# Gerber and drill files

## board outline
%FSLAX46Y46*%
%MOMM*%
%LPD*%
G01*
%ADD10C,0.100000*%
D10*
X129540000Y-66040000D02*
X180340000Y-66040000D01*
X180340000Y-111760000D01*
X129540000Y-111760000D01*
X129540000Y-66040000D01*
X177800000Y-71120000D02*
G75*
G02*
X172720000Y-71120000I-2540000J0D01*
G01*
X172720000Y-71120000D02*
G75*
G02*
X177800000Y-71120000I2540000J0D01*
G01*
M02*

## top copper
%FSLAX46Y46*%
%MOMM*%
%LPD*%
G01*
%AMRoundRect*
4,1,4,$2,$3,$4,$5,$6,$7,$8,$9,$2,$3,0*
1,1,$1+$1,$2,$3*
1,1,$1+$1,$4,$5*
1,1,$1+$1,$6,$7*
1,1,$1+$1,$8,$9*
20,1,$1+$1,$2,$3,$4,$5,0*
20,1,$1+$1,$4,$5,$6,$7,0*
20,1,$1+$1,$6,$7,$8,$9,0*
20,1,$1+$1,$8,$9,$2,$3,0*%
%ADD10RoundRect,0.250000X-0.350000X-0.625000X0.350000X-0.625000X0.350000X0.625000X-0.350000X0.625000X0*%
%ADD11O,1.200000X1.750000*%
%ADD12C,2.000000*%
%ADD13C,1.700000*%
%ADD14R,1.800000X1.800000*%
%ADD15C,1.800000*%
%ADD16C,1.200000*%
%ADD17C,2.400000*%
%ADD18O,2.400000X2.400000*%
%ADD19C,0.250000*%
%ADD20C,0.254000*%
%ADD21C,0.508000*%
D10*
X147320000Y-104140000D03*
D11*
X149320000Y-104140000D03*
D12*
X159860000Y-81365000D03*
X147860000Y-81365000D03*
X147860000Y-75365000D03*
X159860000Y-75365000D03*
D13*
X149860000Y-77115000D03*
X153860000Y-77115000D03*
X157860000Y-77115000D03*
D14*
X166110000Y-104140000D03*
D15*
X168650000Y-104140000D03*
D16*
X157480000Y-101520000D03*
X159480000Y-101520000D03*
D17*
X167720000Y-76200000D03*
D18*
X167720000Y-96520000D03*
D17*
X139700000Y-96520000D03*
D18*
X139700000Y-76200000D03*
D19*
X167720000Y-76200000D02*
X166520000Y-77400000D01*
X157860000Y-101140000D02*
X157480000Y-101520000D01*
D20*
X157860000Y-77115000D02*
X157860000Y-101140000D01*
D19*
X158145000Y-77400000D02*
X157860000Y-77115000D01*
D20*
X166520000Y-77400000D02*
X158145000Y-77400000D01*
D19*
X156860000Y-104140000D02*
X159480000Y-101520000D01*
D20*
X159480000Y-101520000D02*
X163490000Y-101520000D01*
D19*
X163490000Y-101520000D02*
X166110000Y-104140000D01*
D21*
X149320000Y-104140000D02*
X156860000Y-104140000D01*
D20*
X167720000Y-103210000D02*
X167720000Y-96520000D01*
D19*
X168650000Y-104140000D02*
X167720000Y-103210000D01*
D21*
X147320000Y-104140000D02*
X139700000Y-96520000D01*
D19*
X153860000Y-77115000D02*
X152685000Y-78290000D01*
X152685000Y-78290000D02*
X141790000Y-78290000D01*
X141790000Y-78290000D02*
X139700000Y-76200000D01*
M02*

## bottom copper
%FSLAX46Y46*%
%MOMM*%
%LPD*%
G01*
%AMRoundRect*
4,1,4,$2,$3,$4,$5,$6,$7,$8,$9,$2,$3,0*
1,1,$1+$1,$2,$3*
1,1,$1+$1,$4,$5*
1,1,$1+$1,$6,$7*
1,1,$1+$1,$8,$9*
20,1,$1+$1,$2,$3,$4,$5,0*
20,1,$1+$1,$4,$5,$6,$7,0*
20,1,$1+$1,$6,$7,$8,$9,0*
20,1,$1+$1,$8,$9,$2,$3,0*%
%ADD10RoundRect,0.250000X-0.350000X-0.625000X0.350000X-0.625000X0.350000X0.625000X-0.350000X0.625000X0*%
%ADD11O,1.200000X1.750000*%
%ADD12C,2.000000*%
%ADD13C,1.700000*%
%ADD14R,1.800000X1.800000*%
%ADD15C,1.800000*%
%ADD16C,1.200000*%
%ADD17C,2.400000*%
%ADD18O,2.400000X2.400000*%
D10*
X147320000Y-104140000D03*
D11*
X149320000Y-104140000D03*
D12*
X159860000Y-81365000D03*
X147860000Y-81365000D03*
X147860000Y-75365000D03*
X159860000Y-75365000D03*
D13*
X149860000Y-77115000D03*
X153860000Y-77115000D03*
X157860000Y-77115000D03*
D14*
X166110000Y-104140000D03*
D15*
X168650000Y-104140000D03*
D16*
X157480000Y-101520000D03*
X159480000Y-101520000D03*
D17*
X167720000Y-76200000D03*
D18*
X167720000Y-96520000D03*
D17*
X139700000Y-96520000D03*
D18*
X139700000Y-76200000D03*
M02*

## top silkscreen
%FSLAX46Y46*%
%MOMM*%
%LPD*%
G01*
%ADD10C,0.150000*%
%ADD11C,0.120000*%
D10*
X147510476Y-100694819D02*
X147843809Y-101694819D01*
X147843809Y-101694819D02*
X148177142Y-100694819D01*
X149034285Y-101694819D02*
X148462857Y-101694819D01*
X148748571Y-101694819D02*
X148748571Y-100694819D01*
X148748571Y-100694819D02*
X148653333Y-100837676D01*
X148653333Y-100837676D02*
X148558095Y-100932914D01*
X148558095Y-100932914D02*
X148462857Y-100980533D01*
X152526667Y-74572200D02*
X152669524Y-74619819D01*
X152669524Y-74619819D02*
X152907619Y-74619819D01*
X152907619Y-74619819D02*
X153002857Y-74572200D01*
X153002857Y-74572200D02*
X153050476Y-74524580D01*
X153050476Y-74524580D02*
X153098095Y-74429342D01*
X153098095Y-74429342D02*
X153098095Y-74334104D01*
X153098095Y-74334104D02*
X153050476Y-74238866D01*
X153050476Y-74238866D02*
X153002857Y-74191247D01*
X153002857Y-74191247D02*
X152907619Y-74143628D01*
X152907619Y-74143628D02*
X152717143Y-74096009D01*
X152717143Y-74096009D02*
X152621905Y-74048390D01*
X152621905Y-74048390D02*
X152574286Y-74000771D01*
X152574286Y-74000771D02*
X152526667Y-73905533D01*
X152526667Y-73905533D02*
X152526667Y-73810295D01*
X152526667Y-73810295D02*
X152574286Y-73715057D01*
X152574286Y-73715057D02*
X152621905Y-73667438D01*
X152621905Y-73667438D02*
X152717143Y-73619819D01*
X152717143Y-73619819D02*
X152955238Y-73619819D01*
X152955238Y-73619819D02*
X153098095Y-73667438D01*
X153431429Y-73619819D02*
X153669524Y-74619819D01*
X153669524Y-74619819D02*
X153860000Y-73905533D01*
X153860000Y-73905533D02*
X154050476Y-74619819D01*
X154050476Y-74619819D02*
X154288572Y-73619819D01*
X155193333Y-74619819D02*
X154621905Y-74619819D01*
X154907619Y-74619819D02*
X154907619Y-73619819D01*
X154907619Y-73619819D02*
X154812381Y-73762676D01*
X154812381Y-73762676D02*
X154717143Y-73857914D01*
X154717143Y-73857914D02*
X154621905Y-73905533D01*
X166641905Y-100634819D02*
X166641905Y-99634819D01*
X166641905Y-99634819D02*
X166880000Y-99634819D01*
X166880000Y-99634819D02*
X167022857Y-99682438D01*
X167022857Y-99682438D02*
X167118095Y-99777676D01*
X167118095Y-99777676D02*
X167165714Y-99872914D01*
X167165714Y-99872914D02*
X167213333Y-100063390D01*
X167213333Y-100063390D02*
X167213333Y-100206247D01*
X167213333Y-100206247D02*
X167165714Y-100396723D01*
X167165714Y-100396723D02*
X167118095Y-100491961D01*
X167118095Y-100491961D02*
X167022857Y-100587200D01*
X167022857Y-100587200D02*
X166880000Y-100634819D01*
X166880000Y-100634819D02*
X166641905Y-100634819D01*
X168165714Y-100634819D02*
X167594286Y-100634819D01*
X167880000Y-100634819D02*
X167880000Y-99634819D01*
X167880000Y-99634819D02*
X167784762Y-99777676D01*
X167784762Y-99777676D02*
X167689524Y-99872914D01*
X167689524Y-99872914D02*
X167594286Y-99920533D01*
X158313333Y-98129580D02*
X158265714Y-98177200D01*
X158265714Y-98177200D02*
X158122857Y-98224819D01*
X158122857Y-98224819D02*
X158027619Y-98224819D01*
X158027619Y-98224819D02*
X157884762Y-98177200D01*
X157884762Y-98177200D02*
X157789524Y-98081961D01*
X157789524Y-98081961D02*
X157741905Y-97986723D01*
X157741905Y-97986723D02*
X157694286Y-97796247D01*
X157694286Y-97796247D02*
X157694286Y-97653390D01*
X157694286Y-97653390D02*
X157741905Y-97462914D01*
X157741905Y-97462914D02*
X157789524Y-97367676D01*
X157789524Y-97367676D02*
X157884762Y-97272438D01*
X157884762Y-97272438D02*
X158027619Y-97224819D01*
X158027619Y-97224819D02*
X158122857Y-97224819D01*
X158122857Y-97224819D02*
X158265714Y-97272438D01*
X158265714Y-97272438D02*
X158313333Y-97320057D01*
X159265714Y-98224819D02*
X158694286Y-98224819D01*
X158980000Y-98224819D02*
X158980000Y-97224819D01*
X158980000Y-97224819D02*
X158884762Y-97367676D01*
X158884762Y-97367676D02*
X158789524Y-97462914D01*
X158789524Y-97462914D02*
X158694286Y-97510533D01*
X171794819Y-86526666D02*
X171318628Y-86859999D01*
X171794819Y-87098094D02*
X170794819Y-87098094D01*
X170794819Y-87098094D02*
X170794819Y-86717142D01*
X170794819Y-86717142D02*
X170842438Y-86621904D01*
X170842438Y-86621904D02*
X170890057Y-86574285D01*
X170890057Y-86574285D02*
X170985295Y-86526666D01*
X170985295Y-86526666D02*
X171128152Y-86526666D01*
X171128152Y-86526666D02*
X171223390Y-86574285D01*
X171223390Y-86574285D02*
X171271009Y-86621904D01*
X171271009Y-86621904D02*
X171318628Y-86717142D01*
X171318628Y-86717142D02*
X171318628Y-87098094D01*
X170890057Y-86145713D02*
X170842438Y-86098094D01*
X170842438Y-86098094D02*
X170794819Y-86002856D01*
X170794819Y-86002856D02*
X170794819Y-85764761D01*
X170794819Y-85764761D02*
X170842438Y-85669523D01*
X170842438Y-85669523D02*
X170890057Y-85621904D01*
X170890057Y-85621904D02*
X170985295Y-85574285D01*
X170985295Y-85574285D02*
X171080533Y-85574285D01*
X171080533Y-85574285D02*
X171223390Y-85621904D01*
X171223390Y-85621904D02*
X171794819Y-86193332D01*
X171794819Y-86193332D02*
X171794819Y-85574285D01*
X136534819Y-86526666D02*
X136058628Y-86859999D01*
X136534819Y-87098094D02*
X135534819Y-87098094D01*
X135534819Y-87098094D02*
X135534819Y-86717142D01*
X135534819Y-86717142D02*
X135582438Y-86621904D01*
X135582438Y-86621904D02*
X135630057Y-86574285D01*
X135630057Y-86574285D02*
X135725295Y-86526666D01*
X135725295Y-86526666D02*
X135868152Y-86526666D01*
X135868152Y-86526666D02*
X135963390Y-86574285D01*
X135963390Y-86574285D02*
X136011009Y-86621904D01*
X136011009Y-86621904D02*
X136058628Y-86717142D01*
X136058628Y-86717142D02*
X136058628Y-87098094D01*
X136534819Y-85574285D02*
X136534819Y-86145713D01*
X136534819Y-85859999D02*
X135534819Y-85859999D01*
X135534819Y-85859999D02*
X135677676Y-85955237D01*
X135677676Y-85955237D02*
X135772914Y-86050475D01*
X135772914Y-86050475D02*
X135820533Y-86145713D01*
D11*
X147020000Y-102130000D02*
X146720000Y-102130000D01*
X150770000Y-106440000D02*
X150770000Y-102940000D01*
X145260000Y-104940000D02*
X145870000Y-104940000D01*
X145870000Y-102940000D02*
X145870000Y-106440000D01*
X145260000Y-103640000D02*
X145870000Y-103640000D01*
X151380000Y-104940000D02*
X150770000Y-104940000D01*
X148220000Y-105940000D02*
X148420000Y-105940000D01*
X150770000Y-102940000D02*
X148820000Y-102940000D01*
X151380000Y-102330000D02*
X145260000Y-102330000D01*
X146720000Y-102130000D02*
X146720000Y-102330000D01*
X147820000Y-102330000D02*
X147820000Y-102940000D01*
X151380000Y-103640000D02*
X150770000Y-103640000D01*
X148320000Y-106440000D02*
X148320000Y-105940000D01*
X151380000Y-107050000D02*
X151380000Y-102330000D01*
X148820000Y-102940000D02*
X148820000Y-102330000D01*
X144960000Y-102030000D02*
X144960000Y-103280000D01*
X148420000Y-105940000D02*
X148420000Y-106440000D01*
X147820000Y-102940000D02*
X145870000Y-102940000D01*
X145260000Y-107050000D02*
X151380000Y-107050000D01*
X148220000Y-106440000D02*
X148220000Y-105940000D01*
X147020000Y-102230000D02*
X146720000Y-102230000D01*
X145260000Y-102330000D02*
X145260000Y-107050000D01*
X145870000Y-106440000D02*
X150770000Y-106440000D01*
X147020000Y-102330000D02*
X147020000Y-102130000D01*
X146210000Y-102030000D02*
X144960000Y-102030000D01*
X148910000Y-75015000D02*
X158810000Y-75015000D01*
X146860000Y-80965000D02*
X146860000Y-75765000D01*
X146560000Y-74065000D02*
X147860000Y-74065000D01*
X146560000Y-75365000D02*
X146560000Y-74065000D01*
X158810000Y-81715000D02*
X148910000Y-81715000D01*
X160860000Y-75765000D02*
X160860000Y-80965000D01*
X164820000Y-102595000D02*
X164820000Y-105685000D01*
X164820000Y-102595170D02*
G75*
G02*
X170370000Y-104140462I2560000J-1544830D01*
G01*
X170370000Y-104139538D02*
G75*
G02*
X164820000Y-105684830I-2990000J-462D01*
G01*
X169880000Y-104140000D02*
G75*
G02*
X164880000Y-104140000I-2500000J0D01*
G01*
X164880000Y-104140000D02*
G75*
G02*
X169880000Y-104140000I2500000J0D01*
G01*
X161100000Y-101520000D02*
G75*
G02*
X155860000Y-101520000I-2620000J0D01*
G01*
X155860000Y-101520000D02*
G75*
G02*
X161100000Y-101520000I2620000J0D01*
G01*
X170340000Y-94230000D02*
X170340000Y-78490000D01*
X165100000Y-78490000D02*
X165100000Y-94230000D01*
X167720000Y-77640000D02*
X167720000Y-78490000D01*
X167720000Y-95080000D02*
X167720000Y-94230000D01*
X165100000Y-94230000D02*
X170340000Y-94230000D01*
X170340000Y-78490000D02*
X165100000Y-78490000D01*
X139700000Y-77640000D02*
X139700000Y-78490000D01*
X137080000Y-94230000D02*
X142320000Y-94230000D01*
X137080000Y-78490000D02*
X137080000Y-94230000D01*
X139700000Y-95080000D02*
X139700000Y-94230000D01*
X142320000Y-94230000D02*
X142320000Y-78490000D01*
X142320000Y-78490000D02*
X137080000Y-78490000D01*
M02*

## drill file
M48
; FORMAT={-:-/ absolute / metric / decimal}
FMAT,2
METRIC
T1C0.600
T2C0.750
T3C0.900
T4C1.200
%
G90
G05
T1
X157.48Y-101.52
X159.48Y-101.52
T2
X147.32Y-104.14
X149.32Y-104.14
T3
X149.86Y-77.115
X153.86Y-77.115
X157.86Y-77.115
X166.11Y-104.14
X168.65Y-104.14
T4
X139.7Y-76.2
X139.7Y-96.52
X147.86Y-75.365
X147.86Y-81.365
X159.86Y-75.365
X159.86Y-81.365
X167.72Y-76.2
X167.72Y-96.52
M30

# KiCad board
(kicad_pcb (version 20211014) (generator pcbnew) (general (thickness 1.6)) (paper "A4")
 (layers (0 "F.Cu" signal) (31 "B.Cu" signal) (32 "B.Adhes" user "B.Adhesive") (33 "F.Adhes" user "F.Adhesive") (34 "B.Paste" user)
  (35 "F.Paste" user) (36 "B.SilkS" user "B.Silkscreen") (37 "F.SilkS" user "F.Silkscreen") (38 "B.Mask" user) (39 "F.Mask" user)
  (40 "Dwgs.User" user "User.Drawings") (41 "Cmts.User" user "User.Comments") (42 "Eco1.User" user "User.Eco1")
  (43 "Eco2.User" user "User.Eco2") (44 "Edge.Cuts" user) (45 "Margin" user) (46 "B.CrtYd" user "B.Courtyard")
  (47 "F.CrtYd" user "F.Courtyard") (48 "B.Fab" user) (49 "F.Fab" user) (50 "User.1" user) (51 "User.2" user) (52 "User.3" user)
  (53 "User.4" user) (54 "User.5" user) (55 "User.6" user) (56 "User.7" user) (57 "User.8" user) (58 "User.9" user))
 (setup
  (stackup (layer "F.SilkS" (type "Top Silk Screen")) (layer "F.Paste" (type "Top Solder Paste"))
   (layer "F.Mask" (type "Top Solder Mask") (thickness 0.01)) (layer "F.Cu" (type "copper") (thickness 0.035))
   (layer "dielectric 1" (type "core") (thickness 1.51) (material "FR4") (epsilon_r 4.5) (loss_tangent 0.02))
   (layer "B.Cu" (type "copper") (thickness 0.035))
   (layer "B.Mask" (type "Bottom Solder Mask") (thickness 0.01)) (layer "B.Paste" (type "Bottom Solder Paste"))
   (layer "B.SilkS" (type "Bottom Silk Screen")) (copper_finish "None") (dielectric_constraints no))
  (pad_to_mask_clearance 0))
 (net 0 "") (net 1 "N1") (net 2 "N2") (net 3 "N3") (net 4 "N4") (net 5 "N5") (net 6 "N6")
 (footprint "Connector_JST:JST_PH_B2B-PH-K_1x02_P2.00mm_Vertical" (layer "F.Cu") (at 147.32 104.14)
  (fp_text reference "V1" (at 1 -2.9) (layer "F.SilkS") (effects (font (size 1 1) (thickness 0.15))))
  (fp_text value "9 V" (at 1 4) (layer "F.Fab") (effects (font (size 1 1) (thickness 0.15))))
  (fp_line (start -0.3 -2.01) (end -0.6 -2.01) (layer "F.SilkS") (width 0.12))
  (fp_line (start 3.45 2.3) (end 3.45 -1.2) (layer "F.SilkS") (width 0.12))
  (fp_line (start -2.06 0.8) (end -1.45 0.8) (layer "F.SilkS") (width 0.12))
  (fp_line (start -1.45 -1.2) (end -1.45 2.3) (layer "F.SilkS") (width 0.12))
  (fp_line (start -2.06 -0.5) (end -1.45 -0.5) (layer "F.SilkS") (width 0.12))
  (fp_line (start 4.06 0.8) (end 3.45 0.8) (layer "F.SilkS") (width 0.12))
  (fp_line (start 0.9 1.8) (end 1.1 1.8) (layer "F.SilkS") (width 0.12))
  (fp_line (start 3.45 -1.2) (end 1.5 -1.2) (layer "F.SilkS") (width 0.12))
  (fp_line (start 4.06 -1.81) (end -2.06 -1.81) (layer "F.SilkS") (width 0.12))
  (fp_line (start -0.6 -2.01) (end -0.6 -1.81) (layer "F.SilkS") (width 0.12))
  (fp_line (start 0.5 -1.81) (end 0.5 -1.2) (layer "F.SilkS") (width 0.12))
  (fp_line (start 4.06 -0.5) (end 3.45 -0.5) (layer "F.SilkS") (width 0.12))
  (fp_line (start 1 2.3) (end 1 1.8) (layer "F.SilkS") (width 0.12))
  (fp_line (start 4.06 2.91) (end 4.06 -1.81) (layer "F.SilkS") (width 0.12))
  (fp_line (start 1.5 -1.2) (end 1.5 -1.81) (layer "F.SilkS") (width 0.12))
  (fp_line (start -2.36 -2.11) (end -2.36 -0.86) (layer "F.SilkS") (width 0.12))
  (fp_line (start 1.1 1.8) (end 1.1 2.3) (layer "F.SilkS") (width 0.12))
  (fp_line (start 0.5 -1.2) (end -1.45 -1.2) (layer "F.SilkS") (width 0.12))
  (fp_line (start -2.06 2.91) (end 4.06 2.91) (layer "F.SilkS") (width 0.12))
  (fp_line (start 0.9 2.3) (end 0.9 1.8) (layer "F.SilkS") (width 0.12))
  (fp_line (start -0.3 -1.91) (end -0.6 -1.91) (layer "F.SilkS") (width 0.12))
  (fp_line (start -2.06 -1.81) (end -2.06 2.91) (layer "F.SilkS") (width 0.12))
  (fp_line (start -1.45 2.3) (end 3.45 2.3) (layer "F.SilkS") (width 0.12))
  (fp_line (start -0.3 -1.81) (end -0.3 -2.01) (layer "F.SilkS") (width 0.12))
  (fp_line (start -1.11 -2.11) (end -2.36 -2.11) (layer "F.SilkS") (width 0.12))
  (pad "1" thru_hole roundrect (at 0 0) (size 1.2 1.75) (drill 0.75) (layers *.Cu *.Mask) (roundrect_rratio 0.208333) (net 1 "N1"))
  (pad "2" thru_hole oval (at 2 0) (size 1.2 1.75) (drill 0.75) (layers *.Cu *.Mask) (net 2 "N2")))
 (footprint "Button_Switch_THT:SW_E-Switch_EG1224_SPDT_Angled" (layer "F.Cu") (at 149.86 77.115)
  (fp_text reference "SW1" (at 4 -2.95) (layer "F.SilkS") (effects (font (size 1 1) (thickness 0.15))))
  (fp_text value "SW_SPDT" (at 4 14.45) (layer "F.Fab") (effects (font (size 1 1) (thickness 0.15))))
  (fp_line (start -0.95 -2.1) (end 8.95 -2.1) (layer "F.SilkS") (width 0.12))
  (fp_line (start -3 3.85) (end -3 -1.35) (layer "F.SilkS") (width 0.12))
  (fp_line (start -3.3 -3.05) (end -2 -3.05) (layer "F.SilkS") (width 0.12))
  (fp_line (start -3.3 -1.75) (end -3.3 -3.05) (layer "F.SilkS") (width 0.12))
  (fp_line (start 8.95 4.6) (end -0.95 4.6) (layer "F.SilkS") (width 0.12))
  (fp_line (start 11 -1.35) (end 11 3.85) (layer "F.SilkS") (width 0.12))
  (pad "" thru_hole circle (at 10 4.25) (size 2 2) (drill 1.2) (layers *.Cu *.Mask))
  (pad "" thru_hole circle (at -2 4.25) (size 2 2) (drill 1.2) (layers *.Cu *.Mask))
  (pad "" thru_hole circle (at -2 -1.75) (size 2 2) (drill 1.2) (layers *.Cu *.Mask))
  (pad "" thru_hole circle (at 10 -1.75) (size 2 2) (drill 1.2) (layers *.Cu *.Mask))
  (pad "1" thru_hole circle (at 0 0) (size 1.7 1.7) (drill 0.9) (layers *.Cu *.Mask) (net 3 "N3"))
  (pad "2" thru_hole circle (at 4 0) (size 1.7 1.7) (drill 0.9) (layers *.Cu *.Mask) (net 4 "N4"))
  (pad "3" thru_hole circle (at 8 0) (size 1.7 1.7) (drill 0.9) (layers *.Cu *.Mask) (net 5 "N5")))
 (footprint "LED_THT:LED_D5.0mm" (layer "F.Cu") (at 166.11 104.14)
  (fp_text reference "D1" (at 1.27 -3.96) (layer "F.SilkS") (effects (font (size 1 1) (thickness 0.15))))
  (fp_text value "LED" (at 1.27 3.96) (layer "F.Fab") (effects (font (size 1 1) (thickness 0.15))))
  (fp_line (start -1.29 -1.545) (end -1.29 1.545) (layer "F.SilkS") (width 0.12))
  (fp_arc (start -1.29 -1.54483) (mid 2.072002 -2.880433) (end 4.26 0.000462) (layer "F.SilkS") (width 0.12))
  (fp_arc (start 4.26 -0.000462) (mid 2.072002 2.880433) (end -1.29 1.54483) (layer "F.SilkS") (width 0.12))
  (fp_circle (center 1.27 0) (end 3.77 0) (layer "F.SilkS") (width 0.12) (fill none))
  (pad "1" thru_hole rect (at 0 0) (size 1.8 1.8) (drill 0.9) (layers *.Cu *.Mask) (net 2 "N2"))
  (pad "2" thru_hole circle (at 2.54 0) (size 1.8 1.8) (drill 0.9) (layers *.Cu *.Mask) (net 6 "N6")))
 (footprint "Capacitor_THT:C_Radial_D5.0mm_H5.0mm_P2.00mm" (layer "F.Cu") (at 157.48 101.52)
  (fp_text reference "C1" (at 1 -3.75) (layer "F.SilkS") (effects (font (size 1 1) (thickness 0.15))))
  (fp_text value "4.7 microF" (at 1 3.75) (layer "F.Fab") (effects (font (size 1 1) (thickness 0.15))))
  (fp_circle (center 1 0) (end 3.62 0) (layer "F.SilkS") (width 0.12) (fill none))
  (pad "1" thru_hole circle (at 0 0) (size 1.2 1.2) (drill 0.6) (layers *.Cu *.Mask) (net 5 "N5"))
  (pad "2" thru_hole circle (at 2 0) (size 1.2 1.2) (drill 0.6) (layers *.Cu *.Mask) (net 2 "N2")))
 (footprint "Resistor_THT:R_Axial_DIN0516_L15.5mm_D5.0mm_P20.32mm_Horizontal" (layer "F.Cu") (at 167.72 76.2 -90)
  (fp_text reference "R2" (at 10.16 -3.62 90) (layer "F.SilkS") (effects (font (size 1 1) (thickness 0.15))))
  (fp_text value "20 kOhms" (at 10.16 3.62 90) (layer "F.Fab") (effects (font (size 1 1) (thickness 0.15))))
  (fp_line (start 18.03 -2.62) (end 2.29 -2.62) (layer "F.SilkS") (width 0.12))
  (fp_line (start 2.29 2.62) (end 18.03 2.62) (layer "F.SilkS") (width 0.12))
  (fp_line (start 1.44 0) (end 2.29 0) (layer "F.SilkS") (width 0.12))
  (fp_line (start 18.88 0) (end 18.03 0) (layer "F.SilkS") (width 0.12))
  (fp_line (start 18.03 2.62) (end 18.03 -2.62) (layer "F.SilkS") (width 0.12))
  (fp_line (start 2.29 -2.62) (end 2.29 2.62) (layer "F.SilkS") (width 0.12))
  (pad "1" thru_hole circle (at 0 0 270) (size 2.4 2.4) (drill 1.2) (layers *.Cu *.Mask) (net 5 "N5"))
  (pad "2" thru_hole oval (at 20.32 0 270) (size 2.4 2.4) (drill 1.2) (layers *.Cu *.Mask) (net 6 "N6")))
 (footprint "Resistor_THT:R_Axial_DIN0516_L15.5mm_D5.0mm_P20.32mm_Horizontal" (layer "F.Cu") (at 139.7 96.52 90)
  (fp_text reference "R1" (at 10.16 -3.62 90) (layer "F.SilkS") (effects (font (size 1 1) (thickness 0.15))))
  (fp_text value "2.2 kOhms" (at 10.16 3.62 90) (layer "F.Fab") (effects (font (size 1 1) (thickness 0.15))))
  (fp_line (start 18.88 0) (end 18.03 0) (layer "F.SilkS") (width 0.12))
  (fp_line (start 2.29 -2.62) (end 2.29 2.62) (layer "F.SilkS") (width 0.12))
  (fp_line (start 18.03 -2.62) (end 2.29 -2.62) (layer "F.SilkS") (width 0.12))
  (fp_line (start 1.44 0) (end 2.29 0) (layer "F.SilkS") (width 0.12))
  (fp_line (start 2.29 2.62) (end 18.03 2.62) (layer "F.SilkS") (width 0.12))
  (fp_line (start 18.03 2.62) (end 18.03 -2.62) (layer "F.SilkS") (width 0.12))
  (pad "1" thru_hole circle (at 0 0 90) (size 2.4 2.4) (drill 1.2) (layers *.Cu *.Mask) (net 1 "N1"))
  (pad "2" thru_hole oval (at 20.32 0 90) (size 2.4 2.4) (drill 1.2) (layers *.Cu *.Mask) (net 4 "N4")))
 (gr_rect (start 129.54 66.04) (end 180.34 111.76) (layer "Edge.Cuts") (width 0.1) (fill none))
 (gr_circle (center 175.26 71.12) (end 177.8 71.12) (layer "Edge.Cuts") (width 0.1) (fill none))
 (segment (start 167.72 76.2) (end 166.52 77.4) (width 0.25) (layer "F.Cu") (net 5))
 (segment (start 157.86 101.14) (end 157.48 101.52) (width 0.25) (layer "F.Cu") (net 5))
 (segment (start 157.86 77.115) (end 157.86 101.14) (width 0.254) (layer "F.Cu") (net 5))
 (segment (start 158.145 77.4) (end 157.86 77.115) (width 0.25) (layer "F.Cu") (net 5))
 (segment (start 166.52 77.4) (end 158.145 77.4) (width 0.254) (layer "F.Cu") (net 5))
 (segment (start 156.86 104.14) (end 159.48 101.52) (width 0.25) (layer "F.Cu") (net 2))
 (segment (start 159.48 101.52) (end 163.49 101.52) (width 0.254) (layer "F.Cu") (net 2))
 (segment (start 163.49 101.52) (end 166.11 104.14) (width 0.25) (layer "F.Cu") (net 2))
 (segment (start 149.32 104.14) (end 156.86 104.14) (width 0.508) (layer "F.Cu") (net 2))
 (segment (start 167.72 103.21) (end 167.72 96.52) (width 0.254) (layer "F.Cu") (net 6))
 (segment (start 168.65 104.14) (end 167.72 103.21) (width 0.25) (layer "F.Cu") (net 6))
 (segment (start 147.32 104.14) (end 139.7 96.52) (width 0.508) (layer "F.Cu") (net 1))
 (segment (start 153.86 77.115) (end 152.685 78.29) (width 0.25) (layer "F.Cu") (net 4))
 (segment (start 152.685 78.29) (end 141.79 78.29) (width 0.25) (layer "F.Cu") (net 4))
 (segment (start 141.79 78.29) (end 139.7 76.2) (width 0.25) (layer "F.Cu") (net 4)))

